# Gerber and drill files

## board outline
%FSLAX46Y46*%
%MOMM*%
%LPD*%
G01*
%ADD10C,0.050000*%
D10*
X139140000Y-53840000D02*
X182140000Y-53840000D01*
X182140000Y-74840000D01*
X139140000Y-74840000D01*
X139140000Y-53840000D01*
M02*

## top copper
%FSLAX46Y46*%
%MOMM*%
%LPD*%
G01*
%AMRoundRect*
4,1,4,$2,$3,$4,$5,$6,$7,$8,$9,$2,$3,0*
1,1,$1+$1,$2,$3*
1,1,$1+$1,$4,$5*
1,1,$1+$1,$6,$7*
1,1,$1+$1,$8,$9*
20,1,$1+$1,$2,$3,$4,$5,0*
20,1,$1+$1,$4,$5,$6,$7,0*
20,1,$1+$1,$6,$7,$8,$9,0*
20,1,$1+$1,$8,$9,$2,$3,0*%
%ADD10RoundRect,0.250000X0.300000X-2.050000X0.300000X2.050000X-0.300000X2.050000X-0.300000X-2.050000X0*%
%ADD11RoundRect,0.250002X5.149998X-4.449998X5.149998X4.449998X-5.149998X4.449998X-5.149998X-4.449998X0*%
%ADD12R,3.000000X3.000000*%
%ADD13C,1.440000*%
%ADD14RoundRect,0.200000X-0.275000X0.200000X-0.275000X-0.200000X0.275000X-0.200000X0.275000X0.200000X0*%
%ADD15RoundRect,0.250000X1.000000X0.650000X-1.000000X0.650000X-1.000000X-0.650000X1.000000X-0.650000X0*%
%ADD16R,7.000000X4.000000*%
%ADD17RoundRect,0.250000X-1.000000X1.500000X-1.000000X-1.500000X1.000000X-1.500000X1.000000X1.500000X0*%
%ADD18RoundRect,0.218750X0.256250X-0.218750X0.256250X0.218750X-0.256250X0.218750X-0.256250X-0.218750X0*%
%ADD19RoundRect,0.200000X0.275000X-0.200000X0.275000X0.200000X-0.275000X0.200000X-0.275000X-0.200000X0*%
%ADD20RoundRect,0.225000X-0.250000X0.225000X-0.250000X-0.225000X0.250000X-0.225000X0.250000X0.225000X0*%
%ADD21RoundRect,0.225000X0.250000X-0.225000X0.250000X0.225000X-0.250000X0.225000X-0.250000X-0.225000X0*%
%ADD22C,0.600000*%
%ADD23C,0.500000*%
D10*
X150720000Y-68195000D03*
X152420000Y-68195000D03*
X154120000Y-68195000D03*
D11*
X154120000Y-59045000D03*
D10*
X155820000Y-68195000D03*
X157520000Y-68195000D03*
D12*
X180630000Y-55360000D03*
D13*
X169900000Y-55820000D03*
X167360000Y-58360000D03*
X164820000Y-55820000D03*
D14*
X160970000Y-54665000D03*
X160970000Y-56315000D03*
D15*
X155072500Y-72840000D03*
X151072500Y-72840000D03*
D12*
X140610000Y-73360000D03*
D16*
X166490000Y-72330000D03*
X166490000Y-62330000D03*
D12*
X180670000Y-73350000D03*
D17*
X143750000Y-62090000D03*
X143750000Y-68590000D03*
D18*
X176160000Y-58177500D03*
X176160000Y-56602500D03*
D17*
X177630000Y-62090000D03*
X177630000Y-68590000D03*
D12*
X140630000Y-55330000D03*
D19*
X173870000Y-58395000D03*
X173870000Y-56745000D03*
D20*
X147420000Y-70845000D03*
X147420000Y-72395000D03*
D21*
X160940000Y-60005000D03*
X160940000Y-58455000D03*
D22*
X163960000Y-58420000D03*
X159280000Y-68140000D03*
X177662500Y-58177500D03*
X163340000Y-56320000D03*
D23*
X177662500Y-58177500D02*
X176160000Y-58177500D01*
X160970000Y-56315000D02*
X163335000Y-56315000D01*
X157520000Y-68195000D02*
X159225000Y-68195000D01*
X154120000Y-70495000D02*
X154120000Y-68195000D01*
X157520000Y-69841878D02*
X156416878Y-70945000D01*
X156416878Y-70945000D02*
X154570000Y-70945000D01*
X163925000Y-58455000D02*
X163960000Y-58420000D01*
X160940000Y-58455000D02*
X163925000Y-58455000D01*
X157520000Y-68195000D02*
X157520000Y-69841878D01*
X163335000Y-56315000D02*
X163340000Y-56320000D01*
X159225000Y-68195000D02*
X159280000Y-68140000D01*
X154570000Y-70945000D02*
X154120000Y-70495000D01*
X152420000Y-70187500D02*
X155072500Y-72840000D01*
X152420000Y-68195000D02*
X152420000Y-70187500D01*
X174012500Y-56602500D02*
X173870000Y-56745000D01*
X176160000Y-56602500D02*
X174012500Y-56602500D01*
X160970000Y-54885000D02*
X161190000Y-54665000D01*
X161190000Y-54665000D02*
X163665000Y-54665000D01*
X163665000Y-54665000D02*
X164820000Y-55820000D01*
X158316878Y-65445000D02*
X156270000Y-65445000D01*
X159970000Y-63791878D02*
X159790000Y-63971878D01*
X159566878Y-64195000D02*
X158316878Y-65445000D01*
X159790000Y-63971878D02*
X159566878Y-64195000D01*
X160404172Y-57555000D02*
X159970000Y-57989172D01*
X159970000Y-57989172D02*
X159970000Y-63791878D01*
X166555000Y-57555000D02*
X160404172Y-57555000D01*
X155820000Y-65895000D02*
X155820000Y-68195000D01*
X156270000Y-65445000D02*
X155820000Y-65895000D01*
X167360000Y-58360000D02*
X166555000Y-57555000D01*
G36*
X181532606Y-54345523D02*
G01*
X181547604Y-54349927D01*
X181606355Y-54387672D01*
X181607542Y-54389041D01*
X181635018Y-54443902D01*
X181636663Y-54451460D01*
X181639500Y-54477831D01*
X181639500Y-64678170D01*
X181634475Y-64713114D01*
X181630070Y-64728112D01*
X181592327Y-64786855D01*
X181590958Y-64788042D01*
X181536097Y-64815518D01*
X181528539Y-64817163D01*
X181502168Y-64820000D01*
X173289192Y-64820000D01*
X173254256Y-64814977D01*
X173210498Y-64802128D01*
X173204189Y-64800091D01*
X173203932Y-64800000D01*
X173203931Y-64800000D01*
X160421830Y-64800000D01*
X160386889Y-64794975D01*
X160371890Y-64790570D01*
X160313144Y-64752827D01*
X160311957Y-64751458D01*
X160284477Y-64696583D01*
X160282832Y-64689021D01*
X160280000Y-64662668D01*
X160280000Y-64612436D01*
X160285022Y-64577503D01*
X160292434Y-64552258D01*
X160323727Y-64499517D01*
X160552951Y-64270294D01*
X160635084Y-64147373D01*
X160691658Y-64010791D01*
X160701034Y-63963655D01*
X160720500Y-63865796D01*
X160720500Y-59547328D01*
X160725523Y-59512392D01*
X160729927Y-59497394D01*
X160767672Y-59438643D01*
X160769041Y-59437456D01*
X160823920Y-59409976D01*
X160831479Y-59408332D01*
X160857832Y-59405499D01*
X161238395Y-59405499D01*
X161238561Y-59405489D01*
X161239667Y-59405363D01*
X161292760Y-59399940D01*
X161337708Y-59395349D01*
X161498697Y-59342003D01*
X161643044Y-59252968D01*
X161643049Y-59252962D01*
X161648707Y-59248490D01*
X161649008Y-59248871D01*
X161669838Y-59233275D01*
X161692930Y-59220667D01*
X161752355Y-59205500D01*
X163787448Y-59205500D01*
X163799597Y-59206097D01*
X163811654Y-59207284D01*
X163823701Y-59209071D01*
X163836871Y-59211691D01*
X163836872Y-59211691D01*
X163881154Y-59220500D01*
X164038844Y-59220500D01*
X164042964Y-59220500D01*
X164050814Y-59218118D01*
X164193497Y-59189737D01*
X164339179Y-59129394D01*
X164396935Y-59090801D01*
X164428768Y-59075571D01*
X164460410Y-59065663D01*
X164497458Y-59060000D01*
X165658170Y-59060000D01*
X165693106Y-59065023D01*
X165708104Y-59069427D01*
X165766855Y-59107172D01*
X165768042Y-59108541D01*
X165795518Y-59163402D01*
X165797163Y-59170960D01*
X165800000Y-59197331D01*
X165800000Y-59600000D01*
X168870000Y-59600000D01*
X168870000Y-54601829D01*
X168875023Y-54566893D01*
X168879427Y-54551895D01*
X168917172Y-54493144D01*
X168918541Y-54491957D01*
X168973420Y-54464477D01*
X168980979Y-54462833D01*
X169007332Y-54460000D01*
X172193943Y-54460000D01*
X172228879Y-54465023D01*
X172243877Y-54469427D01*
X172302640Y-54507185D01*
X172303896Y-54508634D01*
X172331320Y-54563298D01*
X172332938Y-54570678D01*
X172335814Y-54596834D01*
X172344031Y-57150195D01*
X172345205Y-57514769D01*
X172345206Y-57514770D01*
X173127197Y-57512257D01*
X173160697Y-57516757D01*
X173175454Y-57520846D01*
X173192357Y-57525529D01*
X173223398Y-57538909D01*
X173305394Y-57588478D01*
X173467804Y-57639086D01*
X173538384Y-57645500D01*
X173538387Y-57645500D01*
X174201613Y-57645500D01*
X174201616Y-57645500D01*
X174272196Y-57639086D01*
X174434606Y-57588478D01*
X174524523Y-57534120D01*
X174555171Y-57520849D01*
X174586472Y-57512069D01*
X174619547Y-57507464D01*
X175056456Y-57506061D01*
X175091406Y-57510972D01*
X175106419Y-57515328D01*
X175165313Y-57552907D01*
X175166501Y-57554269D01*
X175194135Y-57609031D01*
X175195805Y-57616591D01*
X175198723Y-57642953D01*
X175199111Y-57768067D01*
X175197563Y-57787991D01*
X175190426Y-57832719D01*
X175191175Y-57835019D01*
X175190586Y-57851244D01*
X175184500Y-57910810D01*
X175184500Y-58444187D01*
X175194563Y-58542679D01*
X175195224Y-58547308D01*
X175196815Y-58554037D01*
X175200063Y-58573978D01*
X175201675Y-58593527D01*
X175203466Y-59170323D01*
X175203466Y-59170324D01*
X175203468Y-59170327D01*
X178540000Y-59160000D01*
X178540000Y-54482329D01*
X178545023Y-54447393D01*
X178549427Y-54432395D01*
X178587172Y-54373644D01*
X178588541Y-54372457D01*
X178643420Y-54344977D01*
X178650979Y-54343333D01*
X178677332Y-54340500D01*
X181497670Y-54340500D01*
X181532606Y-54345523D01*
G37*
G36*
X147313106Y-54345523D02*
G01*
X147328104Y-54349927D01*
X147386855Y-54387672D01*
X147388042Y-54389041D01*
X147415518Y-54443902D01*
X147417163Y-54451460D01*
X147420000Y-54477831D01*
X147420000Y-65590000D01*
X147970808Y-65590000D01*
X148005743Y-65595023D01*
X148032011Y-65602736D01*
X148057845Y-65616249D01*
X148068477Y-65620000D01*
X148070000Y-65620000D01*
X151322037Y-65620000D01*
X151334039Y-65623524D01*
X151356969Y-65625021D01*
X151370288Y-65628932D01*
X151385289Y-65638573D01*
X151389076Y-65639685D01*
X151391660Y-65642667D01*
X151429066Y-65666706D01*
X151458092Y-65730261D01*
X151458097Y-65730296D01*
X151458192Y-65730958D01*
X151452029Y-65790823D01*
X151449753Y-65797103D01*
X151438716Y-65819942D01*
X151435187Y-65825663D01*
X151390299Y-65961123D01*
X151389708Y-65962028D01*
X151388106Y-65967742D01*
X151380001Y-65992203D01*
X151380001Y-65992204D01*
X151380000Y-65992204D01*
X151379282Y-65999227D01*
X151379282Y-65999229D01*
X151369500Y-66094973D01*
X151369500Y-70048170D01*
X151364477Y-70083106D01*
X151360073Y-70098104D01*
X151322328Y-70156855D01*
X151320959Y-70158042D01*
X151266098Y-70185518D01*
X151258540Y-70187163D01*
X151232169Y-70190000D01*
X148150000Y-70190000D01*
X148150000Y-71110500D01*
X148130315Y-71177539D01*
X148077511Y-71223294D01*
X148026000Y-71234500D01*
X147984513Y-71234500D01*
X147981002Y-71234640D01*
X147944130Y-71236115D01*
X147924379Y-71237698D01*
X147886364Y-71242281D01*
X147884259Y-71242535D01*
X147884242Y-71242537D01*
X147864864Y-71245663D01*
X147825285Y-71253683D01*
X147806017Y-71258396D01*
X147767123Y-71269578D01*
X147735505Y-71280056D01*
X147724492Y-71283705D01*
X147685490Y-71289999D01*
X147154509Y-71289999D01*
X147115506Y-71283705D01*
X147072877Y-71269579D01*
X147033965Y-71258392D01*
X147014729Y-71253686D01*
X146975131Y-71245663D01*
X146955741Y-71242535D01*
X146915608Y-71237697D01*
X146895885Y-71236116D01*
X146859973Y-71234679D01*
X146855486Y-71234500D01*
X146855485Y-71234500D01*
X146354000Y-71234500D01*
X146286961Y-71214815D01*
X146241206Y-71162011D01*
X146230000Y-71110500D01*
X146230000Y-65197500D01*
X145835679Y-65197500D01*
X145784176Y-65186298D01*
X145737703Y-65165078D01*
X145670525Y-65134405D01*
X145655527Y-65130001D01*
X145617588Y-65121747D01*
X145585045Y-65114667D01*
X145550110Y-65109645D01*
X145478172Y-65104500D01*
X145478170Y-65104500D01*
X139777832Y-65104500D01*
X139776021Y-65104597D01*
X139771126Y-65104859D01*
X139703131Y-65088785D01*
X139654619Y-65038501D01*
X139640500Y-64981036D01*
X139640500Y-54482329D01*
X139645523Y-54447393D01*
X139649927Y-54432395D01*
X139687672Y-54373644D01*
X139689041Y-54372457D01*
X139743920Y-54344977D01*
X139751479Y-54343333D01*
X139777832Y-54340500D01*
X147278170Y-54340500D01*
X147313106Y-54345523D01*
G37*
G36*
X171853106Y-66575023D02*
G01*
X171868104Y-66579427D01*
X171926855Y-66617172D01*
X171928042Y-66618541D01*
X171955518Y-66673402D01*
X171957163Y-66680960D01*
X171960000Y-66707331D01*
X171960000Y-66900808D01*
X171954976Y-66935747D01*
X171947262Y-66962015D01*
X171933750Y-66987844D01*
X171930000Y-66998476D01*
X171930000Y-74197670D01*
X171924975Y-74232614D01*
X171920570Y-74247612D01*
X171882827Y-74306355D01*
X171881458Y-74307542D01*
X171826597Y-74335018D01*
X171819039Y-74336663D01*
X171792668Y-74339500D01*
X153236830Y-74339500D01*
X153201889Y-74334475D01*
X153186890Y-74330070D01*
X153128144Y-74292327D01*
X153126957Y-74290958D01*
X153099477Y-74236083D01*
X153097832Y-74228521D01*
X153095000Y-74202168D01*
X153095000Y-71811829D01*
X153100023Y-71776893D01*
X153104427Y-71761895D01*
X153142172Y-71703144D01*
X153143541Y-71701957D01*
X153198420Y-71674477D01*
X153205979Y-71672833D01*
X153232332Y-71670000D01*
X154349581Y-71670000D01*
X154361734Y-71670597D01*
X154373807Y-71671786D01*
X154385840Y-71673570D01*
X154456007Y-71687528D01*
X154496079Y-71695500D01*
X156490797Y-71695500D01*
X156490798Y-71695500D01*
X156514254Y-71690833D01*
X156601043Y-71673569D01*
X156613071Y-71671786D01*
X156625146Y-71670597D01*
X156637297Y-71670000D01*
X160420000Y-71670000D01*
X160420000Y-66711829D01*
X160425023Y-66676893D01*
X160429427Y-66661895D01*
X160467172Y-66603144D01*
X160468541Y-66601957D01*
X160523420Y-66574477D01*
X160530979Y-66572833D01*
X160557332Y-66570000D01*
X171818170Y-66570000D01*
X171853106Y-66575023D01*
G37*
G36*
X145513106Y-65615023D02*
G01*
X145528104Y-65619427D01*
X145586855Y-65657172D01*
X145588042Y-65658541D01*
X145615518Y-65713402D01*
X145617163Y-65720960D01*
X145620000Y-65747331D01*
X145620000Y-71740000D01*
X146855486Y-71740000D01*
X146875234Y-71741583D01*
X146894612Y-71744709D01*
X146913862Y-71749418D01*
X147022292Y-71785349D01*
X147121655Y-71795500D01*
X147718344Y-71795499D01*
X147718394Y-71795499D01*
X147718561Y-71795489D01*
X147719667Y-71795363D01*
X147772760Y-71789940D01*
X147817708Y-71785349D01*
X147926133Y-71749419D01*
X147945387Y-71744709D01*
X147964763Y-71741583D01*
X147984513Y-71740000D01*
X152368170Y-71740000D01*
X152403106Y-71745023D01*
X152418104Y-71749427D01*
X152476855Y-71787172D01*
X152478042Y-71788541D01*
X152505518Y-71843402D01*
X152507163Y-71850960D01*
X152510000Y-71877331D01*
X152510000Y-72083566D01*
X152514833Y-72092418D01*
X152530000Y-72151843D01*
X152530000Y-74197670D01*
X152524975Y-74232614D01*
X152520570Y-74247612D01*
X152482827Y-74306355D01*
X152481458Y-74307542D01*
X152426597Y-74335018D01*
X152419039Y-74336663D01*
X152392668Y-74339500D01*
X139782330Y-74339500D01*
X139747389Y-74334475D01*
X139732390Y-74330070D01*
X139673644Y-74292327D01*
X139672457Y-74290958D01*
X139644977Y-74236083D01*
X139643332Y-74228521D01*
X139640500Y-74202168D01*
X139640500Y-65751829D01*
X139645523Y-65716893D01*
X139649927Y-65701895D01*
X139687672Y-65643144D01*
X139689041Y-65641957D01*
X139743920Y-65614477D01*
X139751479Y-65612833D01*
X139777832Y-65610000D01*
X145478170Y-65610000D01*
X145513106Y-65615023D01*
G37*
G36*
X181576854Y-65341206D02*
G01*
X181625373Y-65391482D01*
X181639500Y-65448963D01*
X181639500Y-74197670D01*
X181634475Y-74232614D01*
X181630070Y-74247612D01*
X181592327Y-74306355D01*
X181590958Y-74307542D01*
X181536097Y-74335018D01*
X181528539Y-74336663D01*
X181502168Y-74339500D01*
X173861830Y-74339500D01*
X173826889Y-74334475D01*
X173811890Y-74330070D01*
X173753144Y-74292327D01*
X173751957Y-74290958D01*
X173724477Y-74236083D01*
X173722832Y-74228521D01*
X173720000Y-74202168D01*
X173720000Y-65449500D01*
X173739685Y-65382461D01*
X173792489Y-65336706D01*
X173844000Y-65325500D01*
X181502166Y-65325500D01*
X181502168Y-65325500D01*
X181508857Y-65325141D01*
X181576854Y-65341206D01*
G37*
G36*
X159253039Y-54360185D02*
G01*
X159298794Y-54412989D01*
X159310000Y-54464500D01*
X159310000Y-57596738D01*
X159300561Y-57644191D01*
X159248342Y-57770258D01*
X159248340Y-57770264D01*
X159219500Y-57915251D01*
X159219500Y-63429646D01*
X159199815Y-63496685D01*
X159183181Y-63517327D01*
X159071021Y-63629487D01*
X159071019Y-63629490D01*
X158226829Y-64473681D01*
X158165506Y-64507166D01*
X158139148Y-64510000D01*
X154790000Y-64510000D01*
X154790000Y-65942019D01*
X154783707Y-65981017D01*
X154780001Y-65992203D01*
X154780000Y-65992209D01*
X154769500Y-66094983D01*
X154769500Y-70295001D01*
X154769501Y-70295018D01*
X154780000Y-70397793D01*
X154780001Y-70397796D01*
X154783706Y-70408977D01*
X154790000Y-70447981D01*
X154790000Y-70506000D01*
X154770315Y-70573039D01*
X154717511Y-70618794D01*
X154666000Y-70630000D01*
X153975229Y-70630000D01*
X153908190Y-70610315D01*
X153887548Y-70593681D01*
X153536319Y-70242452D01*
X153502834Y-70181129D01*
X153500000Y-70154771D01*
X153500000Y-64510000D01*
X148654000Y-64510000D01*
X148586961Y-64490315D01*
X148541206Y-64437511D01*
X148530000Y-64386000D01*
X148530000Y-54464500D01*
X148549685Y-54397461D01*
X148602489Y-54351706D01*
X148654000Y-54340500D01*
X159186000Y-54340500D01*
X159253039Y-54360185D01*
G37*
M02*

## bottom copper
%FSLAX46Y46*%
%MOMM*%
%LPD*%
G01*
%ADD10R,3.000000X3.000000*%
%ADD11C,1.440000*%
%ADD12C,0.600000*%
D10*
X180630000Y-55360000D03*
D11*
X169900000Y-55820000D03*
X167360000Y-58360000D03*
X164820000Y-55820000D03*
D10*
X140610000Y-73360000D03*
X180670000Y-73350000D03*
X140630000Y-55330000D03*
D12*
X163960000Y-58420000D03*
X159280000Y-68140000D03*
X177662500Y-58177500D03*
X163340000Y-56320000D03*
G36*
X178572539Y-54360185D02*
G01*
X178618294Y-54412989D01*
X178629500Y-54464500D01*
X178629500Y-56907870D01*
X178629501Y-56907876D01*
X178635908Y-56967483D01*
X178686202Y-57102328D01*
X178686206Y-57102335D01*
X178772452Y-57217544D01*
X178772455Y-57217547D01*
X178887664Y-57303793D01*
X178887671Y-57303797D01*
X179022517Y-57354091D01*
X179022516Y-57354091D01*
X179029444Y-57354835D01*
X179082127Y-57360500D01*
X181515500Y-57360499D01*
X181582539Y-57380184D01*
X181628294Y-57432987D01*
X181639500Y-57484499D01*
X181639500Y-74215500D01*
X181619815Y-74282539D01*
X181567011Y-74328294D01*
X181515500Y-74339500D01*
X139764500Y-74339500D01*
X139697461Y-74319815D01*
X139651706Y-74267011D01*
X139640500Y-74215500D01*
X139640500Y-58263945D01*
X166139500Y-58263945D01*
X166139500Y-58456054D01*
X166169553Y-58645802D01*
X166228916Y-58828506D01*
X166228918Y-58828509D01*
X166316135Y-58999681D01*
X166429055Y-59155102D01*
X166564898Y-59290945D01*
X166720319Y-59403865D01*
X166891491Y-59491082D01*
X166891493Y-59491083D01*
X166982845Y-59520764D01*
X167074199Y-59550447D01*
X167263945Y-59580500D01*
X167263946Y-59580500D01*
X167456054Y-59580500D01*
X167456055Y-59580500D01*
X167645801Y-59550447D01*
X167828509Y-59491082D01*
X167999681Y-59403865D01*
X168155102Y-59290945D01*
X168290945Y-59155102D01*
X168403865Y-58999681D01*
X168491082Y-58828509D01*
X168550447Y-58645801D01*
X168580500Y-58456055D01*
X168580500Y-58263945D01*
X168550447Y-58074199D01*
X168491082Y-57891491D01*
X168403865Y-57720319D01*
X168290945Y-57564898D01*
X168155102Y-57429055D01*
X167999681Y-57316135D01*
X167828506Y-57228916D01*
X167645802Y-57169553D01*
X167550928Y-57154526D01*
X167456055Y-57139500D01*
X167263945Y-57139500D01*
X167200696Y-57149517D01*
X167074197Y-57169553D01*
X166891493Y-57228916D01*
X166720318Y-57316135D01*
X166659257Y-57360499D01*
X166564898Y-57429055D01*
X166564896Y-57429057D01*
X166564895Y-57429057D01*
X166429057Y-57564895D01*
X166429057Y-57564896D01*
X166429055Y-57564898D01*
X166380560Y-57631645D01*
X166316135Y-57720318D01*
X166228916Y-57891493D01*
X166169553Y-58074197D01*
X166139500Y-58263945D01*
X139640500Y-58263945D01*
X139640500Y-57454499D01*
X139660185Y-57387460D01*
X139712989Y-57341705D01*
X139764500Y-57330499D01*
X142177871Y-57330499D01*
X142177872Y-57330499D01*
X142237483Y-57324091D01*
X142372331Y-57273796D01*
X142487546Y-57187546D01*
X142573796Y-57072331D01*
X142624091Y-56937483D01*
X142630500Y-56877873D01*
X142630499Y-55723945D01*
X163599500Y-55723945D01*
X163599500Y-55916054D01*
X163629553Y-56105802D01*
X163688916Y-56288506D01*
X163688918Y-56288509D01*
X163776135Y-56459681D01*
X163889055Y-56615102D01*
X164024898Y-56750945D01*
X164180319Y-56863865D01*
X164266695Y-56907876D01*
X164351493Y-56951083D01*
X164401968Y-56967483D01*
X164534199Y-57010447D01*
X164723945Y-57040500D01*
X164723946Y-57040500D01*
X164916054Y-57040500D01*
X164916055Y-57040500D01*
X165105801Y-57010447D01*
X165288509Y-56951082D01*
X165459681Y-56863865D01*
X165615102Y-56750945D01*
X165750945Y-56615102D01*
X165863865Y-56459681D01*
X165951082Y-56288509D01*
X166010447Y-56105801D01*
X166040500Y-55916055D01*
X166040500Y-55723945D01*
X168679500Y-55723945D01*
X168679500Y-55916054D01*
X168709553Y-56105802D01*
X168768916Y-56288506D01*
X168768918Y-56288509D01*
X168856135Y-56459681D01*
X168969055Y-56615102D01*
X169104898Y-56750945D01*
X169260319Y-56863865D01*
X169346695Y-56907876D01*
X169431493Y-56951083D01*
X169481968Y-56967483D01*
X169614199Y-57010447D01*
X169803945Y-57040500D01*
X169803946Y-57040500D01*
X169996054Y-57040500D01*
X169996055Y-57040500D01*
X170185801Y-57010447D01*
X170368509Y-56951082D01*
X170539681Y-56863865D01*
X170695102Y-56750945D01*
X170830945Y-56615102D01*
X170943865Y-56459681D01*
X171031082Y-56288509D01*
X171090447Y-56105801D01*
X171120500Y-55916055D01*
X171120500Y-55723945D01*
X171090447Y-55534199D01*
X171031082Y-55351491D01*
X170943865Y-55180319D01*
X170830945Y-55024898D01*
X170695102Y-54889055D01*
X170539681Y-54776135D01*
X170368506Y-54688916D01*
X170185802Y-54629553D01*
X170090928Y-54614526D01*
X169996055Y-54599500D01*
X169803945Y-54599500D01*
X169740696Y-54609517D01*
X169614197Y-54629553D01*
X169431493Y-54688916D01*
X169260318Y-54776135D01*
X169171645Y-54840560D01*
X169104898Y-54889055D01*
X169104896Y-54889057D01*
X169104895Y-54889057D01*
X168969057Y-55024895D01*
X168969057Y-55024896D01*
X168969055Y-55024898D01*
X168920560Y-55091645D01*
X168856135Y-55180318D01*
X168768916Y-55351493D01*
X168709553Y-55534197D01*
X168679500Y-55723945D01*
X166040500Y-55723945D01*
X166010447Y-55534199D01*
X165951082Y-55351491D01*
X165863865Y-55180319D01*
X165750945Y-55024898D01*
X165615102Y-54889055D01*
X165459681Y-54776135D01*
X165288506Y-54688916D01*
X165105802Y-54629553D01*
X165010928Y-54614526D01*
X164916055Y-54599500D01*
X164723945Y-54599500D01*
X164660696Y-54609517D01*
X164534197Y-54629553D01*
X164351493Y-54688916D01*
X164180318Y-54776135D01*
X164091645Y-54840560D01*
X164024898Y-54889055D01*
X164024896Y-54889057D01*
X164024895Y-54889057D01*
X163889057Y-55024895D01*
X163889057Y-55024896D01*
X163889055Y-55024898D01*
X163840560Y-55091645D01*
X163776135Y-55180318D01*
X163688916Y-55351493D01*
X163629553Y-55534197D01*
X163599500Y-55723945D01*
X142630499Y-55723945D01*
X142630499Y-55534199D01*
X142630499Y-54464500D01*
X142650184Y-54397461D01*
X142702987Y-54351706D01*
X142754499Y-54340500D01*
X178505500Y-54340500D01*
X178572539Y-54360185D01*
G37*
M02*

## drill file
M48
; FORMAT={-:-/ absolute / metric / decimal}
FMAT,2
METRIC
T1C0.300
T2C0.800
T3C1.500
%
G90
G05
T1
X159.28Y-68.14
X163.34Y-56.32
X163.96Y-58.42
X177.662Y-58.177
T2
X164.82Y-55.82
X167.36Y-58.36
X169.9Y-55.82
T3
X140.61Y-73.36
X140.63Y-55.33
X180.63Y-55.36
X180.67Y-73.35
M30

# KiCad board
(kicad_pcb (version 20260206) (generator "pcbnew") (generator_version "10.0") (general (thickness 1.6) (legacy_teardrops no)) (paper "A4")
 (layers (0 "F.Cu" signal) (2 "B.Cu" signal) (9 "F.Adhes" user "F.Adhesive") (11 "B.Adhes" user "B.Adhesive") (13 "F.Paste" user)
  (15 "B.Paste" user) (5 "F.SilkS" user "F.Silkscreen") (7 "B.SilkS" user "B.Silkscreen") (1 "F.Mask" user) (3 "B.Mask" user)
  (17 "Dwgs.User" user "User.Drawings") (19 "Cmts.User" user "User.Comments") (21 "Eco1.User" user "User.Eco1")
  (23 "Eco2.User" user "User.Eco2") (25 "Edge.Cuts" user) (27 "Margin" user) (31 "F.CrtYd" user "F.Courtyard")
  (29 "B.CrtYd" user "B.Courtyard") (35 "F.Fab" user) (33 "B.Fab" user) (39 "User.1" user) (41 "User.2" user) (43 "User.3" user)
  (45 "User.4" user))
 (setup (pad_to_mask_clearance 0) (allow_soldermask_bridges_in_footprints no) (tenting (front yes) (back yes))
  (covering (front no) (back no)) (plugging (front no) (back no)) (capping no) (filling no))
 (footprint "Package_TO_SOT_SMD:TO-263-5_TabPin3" (layer "F.Cu") (at 154.12 60.545 90)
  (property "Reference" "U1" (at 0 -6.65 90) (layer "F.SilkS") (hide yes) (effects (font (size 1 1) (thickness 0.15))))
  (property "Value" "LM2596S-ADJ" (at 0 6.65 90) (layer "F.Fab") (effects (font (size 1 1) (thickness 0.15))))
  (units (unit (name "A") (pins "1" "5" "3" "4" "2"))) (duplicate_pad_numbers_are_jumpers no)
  (pad "" smd roundrect (at -0.925 -2.775 90) (size 4.55 5.25) (layers "F.Paste") (roundrect_rratio 0.054945))
  (pad "" smd roundrect (at -0.925 2.775 90) (size 4.55 5.25) (layers "F.Paste") (roundrect_rratio 0.054945))
  (pad "" smd roundrect (at 3.925 -2.775 90) (size 4.55 5.25) (layers "F.Paste") (roundrect_rratio 0.054945))
  (pad "" smd roundrect (at 3.925 2.775 90) (size 4.55 5.25) (layers "F.Paste") (roundrect_rratio 0.054945))
  (pad "1" smd roundrect (at -7.65 -3.4 90) (size 4.6 1.1) (layers "F.Cu" "F.Mask" "F.Paste") (roundrect_rratio 0.227273) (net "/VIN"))
  (pad "2" smd roundrect (at -7.65 -1.7 90) (size 4.6 1.1) (layers "F.Cu" "F.Mask" "F.Paste") (roundrect_rratio 0.227273) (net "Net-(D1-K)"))
  (pad "3" smd roundrect (at -7.65 0 90) (size 4.6 1.1) (layers "F.Cu" "F.Mask" "F.Paste") (roundrect_rratio 0.227273) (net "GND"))
  (pad "3" smd roundrect (at 1.5 0 90) (size 9.4 10.8) (layers "F.Cu" "F.Mask") (roundrect_rratio 0.026596) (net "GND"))
  (pad "4" smd roundrect (at -7.65 1.7 90) (size 4.6 1.1) (layers "F.Cu" "F.Mask" "F.Paste") (roundrect_rratio 0.227273) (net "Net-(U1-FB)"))
  (pad "5" smd roundrect (at -7.65 3.4 90) (size 4.6 1.1) (layers "F.Cu" "F.Mask" "F.Paste") (roundrect_rratio 0.227273) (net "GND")))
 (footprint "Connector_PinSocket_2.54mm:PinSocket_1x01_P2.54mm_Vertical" (layer "F.Cu") (at 180.63 55.36)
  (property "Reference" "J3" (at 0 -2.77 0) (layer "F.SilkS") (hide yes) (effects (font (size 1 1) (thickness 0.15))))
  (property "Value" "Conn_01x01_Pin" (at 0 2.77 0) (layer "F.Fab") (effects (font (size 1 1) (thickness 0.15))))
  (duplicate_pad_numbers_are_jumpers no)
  (pad "1" thru_hole rect (at 0 0) (size 3 3) (drill 1.5) (layers "*.Cu" "*.Mask" "B.Paste") (remove_unused_layers no) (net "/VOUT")))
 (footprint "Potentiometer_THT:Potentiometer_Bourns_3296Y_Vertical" (layer "F.Cu") (at 169.9 55.82)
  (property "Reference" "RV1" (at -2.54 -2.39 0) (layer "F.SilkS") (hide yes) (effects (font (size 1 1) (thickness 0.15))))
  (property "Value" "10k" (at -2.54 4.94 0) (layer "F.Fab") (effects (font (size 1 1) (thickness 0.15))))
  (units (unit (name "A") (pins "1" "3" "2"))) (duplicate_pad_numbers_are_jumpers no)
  (pad "1" thru_hole circle (at 0 0) (size 1.44 1.44) (drill 0.8) (layers "*.Cu" "*.Mask") (remove_unused_layers no) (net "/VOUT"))
  (pad "2" thru_hole circle (at -2.54 2.54) (size 1.44 1.44) (drill 0.8) (layers "*.Cu" "*.Mask") (remove_unused_layers no)
   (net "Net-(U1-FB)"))
  (pad "3" thru_hole circle (at -5.08 0) (size 1.44 1.44) (drill 0.8) (layers "*.Cu" "*.Mask") (remove_unused_layers no)
   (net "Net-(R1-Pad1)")))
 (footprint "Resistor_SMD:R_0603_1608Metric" (layer "F.Cu") (at 160.97 55.49 -90)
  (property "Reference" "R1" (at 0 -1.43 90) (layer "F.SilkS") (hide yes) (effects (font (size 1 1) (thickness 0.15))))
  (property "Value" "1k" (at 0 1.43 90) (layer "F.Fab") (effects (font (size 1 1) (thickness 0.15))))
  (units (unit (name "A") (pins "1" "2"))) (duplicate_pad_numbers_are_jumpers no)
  (pad "1" smd roundrect (at -0.825 0 270) (size 0.8 0.95) (layers "F.Cu" "F.Mask" "F.Paste") (roundrect_rratio 0.25) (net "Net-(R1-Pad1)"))
  (pad "2" smd roundrect (at 0.825 0 270) (size 0.8 0.95) (layers "F.Cu" "F.Mask" "F.Paste") (roundrect_rratio 0.25) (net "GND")))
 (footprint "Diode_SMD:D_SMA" (layer "F.Cu") (at 153.0725 72.84 180)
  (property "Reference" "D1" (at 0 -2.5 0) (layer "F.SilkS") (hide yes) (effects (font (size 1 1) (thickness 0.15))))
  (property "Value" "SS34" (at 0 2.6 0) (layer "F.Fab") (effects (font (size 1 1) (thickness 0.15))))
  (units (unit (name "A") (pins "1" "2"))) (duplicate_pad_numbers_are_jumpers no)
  (pad "1" smd roundrect (at -2 0 180) (size 2.5 1.8) (layers "F.Cu" "F.Mask" "F.Paste") (roundrect_rratio 0.1388888889) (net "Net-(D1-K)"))
  (pad "2" smd roundrect (at 2 0 180) (size 2.5 1.8) (layers "F.Cu" "F.Mask" "F.Paste") (roundrect_rratio 0.1388888889) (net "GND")))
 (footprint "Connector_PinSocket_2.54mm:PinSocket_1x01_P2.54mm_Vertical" (layer "F.Cu") (at 140.61 73.36)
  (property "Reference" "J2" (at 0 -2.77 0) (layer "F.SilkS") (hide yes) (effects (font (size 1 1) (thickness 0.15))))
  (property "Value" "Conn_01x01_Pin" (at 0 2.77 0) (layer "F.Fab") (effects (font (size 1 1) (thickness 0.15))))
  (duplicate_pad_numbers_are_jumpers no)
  (pad "1" thru_hole rect (at 0 0) (size 3 3) (drill 1.5) (layers "*.Cu" "*.Mask") (remove_unused_layers no) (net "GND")))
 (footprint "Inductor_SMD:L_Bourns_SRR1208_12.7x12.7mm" (layer "F.Cu") (at 166.49 67.33 90)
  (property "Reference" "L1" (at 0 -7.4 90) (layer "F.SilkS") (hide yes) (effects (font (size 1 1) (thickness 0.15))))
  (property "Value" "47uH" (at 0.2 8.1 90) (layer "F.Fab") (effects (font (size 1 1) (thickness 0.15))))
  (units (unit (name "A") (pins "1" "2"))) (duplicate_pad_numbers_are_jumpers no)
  (pad "1" smd rect (at -5 0 90) (size 4 7) (layers "F.Cu" "F.Mask" "F.Paste") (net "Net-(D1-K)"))
  (pad "2" smd rect (at 5 0 90) (size 4 7) (layers "F.Cu" "F.Mask" "F.Paste") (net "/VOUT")))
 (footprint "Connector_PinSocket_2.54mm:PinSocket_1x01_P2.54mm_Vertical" (layer "F.Cu") (at 180.67 73.35)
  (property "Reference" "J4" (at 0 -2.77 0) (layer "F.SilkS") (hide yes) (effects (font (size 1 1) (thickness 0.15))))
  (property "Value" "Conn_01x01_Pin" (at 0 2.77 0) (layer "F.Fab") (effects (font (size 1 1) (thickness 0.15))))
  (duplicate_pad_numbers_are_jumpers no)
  (pad "1" thru_hole rect (at 0 0) (size 3 3) (drill 1.5) (layers "*.Cu" "*.Mask") (remove_unused_layers no) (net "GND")))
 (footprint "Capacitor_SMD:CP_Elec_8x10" (layer "F.Cu") (at 143.75 65.34 -90)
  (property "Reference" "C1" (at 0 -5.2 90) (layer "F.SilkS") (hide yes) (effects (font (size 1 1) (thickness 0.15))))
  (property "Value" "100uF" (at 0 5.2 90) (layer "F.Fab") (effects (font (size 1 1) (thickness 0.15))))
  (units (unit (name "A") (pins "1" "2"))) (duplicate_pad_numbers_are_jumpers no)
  (pad "1" smd roundrect (at -3.25 0 270) (size 3.5 2.5) (layers "F.Cu" "F.Mask" "F.Paste") (roundrect_rratio 0.1) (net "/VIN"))
  (pad "2" smd roundrect (at 3.25 0 270) (size 3.5 2.5) (layers "F.Cu" "F.Mask" "F.Paste") (roundrect_rratio 0.1) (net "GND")))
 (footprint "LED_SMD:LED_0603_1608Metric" (layer "F.Cu") (at 176.16 57.39 90)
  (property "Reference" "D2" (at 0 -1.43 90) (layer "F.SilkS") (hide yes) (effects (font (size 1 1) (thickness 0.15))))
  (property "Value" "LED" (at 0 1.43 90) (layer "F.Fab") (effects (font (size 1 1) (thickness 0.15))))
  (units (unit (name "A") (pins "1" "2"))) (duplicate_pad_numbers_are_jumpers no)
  (pad "1" smd roundrect (at -0.7875 0 90) (size 0.875 0.95) (layers "F.Cu" "F.Mask" "F.Paste") (roundrect_rratio 0.25) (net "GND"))
  (pad "2" smd roundrect (at 0.7875 0 90) (size 0.875 0.95) (layers "F.Cu" "F.Mask" "F.Paste") (roundrect_rratio 0.25) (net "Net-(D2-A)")))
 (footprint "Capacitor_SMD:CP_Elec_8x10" (layer "F.Cu") (at 177.63 65.34 -90)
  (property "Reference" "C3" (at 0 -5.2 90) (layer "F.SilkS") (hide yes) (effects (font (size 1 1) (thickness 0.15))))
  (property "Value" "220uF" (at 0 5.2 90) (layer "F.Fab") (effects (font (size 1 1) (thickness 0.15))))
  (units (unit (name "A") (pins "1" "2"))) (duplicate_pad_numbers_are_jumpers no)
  (pad "1" smd roundrect (at -3.25 0 270) (size 3.5 2.5) (layers "F.Cu" "F.Mask" "F.Paste") (roundrect_rratio 0.1) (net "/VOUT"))
  (pad "2" smd roundrect (at 3.25 0 270) (size 3.5 2.5) (layers "F.Cu" "F.Mask" "F.Paste") (roundrect_rratio 0.1) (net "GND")))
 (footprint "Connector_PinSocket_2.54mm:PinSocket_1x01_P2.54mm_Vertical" (layer "F.Cu") (at 140.63 55.33)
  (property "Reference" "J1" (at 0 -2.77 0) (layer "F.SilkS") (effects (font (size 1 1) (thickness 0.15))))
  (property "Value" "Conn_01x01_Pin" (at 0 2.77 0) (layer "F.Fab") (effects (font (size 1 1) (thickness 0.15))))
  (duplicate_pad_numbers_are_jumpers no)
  (pad "1" thru_hole rect (at 0 0) (size 3 3) (drill 1.5) (layers "*.Cu" "*.Mask") (remove_unused_layers no) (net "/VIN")))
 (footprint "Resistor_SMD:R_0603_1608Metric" (layer "F.Cu") (at 173.87 57.57 90)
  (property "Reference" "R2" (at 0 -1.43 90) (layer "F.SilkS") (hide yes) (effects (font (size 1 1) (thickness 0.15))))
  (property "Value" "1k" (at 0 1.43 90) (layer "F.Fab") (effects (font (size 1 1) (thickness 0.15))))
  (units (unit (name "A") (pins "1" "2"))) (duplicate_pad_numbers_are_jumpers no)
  (pad "1" smd roundrect (at -0.825 0 90) (size 0.8 0.95) (layers "F.Cu" "F.Mask" "F.Paste") (roundrect_rratio 0.25) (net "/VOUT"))
  (pad "2" smd roundrect (at 0.825 0 90) (size 0.8 0.95) (layers "F.Cu" "F.Mask" "F.Paste") (roundrect_rratio 0.25) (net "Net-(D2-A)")))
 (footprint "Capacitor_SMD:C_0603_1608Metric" (layer "F.Cu") (at 147.42 71.62 -90)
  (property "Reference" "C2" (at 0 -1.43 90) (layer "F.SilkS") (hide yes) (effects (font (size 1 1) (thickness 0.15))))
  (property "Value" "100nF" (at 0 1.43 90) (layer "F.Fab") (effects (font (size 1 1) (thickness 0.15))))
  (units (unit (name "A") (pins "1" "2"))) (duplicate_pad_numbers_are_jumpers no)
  (pad "1" smd roundrect (at -0.775 0 270) (size 0.9 0.95) (layers "F.Cu" "F.Mask" "F.Paste") (roundrect_rratio 0.25) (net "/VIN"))
  (pad "2" smd roundrect (at 0.775 0 270) (size 0.9 0.95) (layers "F.Cu" "F.Mask" "F.Paste") (roundrect_rratio 0.25) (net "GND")))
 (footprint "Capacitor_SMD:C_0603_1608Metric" (layer "F.Cu") (at 160.94 59.23 90)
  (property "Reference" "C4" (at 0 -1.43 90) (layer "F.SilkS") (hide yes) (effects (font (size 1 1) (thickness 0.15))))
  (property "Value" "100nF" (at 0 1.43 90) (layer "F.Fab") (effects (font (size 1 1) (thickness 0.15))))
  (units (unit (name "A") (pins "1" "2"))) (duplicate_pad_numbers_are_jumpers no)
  (pad "1" smd roundrect (at -0.775 0 90) (size 0.9 0.95) (layers "F.Cu" "F.Mask" "F.Paste") (roundrect_rratio 0.25) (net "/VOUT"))
  (pad "2" smd roundrect (at 0.775 0 90) (size 0.9 0.95) (layers "F.Cu" "F.Mask" "F.Paste") (roundrect_rratio 0.25) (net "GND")))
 (gr_rect (start 139.14 53.84) (end 182.14 74.84) (stroke (width 0.05) (type solid)) (fill no) (layer "Edge.Cuts"))
 (segment (start 177.6625 58.1775) (end 176.16 58.1775) (width 0.5) (layer "F.Cu") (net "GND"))
 (segment (start 160.97 56.315) (end 163.335 56.315) (width 0.5) (layer "F.Cu") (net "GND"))
 (segment (start 157.52 68.195) (end 159.225 68.195) (width 0.5) (layer "F.Cu") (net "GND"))
 (segment (start 154.12 70.495) (end 154.12 68.195) (width 0.5) (layer "F.Cu") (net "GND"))
 (segment (start 157.52 69.841878) (end 156.416878 70.945) (width 0.5) (layer "F.Cu") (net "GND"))
 (segment (start 156.416878 70.945) (end 154.57 70.945) (width 0.5) (layer "F.Cu") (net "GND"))
 (segment (start 163.925 58.455) (end 163.96 58.42) (width 0.5) (layer "F.Cu") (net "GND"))
 (segment (start 160.94 58.455) (end 163.925 58.455) (width 0.5) (layer "F.Cu") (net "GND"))
 (segment (start 157.52 68.195) (end 157.52 69.841878) (width 0.5) (layer "F.Cu") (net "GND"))
 (segment (start 163.335 56.315) (end 163.34 56.32) (width 0.5) (layer "F.Cu") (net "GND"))
 (segment (start 159.225 68.195) (end 159.28 68.14) (width 0.5) (layer "F.Cu") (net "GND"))
 (segment (start 154.57 70.945) (end 154.12 70.495) (width 0.5) (layer "F.Cu") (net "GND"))
 (via (at 163.96 58.42) (size 0.6) (drill 0.3) (layers "F.Cu" "B.Cu") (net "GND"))
 (via (at 159.28 68.14) (size 0.6) (drill 0.3) (layers "F.Cu" "B.Cu") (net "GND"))
 (via (at 177.6625 58.1775) (size 0.6) (drill 0.3) (layers "F.Cu" "B.Cu") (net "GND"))
 (via (at 163.34 56.32) (size 0.6) (drill 0.3) (layers "F.Cu" "B.Cu") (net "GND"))
 (segment (start 152.42 70.1875) (end 155.0725 72.84) (width 0.5) (layer "F.Cu") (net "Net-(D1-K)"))
 (segment (start 152.42 68.195) (end 152.42 70.1875) (width 0.5) (layer "F.Cu") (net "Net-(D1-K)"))
 (segment (start 174.0125 56.6025) (end 173.87 56.745) (width 0.5) (layer "F.Cu") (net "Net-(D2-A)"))
 (segment (start 176.16 56.6025) (end 174.0125 56.6025) (width 0.5) (layer "F.Cu") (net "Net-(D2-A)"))
 (segment (start 160.97 54.885) (end 161.19 54.665) (width 0.5) (layer "F.Cu") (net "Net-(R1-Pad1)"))
 (segment (start 161.19 54.665) (end 163.665 54.665) (width 0.5) (layer "F.Cu") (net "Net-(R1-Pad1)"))
 (segment (start 163.665 54.665) (end 164.82 55.82) (width 0.5) (layer "F.Cu") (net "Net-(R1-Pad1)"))
 (segment (start 158.316878 65.445) (end 156.27 65.445) (width 0.5) (layer "F.Cu") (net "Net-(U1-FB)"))
 (segment (start 159.97 63.791878) (end 159.79 63.971878) (width 0.5) (layer "F.Cu") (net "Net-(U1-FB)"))
 (segment (start 159.566878 64.195) (end 158.316878 65.445) (width 0.5) (layer "F.Cu") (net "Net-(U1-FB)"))
 (segment (start 159.79 63.971878) (end 159.566878 64.195) (width 0.5) (layer "F.Cu") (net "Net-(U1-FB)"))
 (segment (start 160.404172 57.555) (end 159.97 57.989172) (width 0.5) (layer "F.Cu") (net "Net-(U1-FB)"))
 (segment (start 159.97 57.989172) (end 159.97 63.791878) (width 0.5) (layer "F.Cu") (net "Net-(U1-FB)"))
 (segment (start 166.555 57.555) (end 160.404172 57.555) (width 0.5) (layer "F.Cu") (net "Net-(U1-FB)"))
 (segment (start 155.82 65.895) (end 155.82 68.195) (width 0.5) (layer "F.Cu") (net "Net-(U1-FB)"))
 (segment (start 156.27 65.445) (end 155.82 65.895) (width 0.5) (layer "F.Cu") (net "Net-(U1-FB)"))
 (segment (start 167.36 58.36) (end 166.555 57.555) (width 0.5) (layer "F.Cu") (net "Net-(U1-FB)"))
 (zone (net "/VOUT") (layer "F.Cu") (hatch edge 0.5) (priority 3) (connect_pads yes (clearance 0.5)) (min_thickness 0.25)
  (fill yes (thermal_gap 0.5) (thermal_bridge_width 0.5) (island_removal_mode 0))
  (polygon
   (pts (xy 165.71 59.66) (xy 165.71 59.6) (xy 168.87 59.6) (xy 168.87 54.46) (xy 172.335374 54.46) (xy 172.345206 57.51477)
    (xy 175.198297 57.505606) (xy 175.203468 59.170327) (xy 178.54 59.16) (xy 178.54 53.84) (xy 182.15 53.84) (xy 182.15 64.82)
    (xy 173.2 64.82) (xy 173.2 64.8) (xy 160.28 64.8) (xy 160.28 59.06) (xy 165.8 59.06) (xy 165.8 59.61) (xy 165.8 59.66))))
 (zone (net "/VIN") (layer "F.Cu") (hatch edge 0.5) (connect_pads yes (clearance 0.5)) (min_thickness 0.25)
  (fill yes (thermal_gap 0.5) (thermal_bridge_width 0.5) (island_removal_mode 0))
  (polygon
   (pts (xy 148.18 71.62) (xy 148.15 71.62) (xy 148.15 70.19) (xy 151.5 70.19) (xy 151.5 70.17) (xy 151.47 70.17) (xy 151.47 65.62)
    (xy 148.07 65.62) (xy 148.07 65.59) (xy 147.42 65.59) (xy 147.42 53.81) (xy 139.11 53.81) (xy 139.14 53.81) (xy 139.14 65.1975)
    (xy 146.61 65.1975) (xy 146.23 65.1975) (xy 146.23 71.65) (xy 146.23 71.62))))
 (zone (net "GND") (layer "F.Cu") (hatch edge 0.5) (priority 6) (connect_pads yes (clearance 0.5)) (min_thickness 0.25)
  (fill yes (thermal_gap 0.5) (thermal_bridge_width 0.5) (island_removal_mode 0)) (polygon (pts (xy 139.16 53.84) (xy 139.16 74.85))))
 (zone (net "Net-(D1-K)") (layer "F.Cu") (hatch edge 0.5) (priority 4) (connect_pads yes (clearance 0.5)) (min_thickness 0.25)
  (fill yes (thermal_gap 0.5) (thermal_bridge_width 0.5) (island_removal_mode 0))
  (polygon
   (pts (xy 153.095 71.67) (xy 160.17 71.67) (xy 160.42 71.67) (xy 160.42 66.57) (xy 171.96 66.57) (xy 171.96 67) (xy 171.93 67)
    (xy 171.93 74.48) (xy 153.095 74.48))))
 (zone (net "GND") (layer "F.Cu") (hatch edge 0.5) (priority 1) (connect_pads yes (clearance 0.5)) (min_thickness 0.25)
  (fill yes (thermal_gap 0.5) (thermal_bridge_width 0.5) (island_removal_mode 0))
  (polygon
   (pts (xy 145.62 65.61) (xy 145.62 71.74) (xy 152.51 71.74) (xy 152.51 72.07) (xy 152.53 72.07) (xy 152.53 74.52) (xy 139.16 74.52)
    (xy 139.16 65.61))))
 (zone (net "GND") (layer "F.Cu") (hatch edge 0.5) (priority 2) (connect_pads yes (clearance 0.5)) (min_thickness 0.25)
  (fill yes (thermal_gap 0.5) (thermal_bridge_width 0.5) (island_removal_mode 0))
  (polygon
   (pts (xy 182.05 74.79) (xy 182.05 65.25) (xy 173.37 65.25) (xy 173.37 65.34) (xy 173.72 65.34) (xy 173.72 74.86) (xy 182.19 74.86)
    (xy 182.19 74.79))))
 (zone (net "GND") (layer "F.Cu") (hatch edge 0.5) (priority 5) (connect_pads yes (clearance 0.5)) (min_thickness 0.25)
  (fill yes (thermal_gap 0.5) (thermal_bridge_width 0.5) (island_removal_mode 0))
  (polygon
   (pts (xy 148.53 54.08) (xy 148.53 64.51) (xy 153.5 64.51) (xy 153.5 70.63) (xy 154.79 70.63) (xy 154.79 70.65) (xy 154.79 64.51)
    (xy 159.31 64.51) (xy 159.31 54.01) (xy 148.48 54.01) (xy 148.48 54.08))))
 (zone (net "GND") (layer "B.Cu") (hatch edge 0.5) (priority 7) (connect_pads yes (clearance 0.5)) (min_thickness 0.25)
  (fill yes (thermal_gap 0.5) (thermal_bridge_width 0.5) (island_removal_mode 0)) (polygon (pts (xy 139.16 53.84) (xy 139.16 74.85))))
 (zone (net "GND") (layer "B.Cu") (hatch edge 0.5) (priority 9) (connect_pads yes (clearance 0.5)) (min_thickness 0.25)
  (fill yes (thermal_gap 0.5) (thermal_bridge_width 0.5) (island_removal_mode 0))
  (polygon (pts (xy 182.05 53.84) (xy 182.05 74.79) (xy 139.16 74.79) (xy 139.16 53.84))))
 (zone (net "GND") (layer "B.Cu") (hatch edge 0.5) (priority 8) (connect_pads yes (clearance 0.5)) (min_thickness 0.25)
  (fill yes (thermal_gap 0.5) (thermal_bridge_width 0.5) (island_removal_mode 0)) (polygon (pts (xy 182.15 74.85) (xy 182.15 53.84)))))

